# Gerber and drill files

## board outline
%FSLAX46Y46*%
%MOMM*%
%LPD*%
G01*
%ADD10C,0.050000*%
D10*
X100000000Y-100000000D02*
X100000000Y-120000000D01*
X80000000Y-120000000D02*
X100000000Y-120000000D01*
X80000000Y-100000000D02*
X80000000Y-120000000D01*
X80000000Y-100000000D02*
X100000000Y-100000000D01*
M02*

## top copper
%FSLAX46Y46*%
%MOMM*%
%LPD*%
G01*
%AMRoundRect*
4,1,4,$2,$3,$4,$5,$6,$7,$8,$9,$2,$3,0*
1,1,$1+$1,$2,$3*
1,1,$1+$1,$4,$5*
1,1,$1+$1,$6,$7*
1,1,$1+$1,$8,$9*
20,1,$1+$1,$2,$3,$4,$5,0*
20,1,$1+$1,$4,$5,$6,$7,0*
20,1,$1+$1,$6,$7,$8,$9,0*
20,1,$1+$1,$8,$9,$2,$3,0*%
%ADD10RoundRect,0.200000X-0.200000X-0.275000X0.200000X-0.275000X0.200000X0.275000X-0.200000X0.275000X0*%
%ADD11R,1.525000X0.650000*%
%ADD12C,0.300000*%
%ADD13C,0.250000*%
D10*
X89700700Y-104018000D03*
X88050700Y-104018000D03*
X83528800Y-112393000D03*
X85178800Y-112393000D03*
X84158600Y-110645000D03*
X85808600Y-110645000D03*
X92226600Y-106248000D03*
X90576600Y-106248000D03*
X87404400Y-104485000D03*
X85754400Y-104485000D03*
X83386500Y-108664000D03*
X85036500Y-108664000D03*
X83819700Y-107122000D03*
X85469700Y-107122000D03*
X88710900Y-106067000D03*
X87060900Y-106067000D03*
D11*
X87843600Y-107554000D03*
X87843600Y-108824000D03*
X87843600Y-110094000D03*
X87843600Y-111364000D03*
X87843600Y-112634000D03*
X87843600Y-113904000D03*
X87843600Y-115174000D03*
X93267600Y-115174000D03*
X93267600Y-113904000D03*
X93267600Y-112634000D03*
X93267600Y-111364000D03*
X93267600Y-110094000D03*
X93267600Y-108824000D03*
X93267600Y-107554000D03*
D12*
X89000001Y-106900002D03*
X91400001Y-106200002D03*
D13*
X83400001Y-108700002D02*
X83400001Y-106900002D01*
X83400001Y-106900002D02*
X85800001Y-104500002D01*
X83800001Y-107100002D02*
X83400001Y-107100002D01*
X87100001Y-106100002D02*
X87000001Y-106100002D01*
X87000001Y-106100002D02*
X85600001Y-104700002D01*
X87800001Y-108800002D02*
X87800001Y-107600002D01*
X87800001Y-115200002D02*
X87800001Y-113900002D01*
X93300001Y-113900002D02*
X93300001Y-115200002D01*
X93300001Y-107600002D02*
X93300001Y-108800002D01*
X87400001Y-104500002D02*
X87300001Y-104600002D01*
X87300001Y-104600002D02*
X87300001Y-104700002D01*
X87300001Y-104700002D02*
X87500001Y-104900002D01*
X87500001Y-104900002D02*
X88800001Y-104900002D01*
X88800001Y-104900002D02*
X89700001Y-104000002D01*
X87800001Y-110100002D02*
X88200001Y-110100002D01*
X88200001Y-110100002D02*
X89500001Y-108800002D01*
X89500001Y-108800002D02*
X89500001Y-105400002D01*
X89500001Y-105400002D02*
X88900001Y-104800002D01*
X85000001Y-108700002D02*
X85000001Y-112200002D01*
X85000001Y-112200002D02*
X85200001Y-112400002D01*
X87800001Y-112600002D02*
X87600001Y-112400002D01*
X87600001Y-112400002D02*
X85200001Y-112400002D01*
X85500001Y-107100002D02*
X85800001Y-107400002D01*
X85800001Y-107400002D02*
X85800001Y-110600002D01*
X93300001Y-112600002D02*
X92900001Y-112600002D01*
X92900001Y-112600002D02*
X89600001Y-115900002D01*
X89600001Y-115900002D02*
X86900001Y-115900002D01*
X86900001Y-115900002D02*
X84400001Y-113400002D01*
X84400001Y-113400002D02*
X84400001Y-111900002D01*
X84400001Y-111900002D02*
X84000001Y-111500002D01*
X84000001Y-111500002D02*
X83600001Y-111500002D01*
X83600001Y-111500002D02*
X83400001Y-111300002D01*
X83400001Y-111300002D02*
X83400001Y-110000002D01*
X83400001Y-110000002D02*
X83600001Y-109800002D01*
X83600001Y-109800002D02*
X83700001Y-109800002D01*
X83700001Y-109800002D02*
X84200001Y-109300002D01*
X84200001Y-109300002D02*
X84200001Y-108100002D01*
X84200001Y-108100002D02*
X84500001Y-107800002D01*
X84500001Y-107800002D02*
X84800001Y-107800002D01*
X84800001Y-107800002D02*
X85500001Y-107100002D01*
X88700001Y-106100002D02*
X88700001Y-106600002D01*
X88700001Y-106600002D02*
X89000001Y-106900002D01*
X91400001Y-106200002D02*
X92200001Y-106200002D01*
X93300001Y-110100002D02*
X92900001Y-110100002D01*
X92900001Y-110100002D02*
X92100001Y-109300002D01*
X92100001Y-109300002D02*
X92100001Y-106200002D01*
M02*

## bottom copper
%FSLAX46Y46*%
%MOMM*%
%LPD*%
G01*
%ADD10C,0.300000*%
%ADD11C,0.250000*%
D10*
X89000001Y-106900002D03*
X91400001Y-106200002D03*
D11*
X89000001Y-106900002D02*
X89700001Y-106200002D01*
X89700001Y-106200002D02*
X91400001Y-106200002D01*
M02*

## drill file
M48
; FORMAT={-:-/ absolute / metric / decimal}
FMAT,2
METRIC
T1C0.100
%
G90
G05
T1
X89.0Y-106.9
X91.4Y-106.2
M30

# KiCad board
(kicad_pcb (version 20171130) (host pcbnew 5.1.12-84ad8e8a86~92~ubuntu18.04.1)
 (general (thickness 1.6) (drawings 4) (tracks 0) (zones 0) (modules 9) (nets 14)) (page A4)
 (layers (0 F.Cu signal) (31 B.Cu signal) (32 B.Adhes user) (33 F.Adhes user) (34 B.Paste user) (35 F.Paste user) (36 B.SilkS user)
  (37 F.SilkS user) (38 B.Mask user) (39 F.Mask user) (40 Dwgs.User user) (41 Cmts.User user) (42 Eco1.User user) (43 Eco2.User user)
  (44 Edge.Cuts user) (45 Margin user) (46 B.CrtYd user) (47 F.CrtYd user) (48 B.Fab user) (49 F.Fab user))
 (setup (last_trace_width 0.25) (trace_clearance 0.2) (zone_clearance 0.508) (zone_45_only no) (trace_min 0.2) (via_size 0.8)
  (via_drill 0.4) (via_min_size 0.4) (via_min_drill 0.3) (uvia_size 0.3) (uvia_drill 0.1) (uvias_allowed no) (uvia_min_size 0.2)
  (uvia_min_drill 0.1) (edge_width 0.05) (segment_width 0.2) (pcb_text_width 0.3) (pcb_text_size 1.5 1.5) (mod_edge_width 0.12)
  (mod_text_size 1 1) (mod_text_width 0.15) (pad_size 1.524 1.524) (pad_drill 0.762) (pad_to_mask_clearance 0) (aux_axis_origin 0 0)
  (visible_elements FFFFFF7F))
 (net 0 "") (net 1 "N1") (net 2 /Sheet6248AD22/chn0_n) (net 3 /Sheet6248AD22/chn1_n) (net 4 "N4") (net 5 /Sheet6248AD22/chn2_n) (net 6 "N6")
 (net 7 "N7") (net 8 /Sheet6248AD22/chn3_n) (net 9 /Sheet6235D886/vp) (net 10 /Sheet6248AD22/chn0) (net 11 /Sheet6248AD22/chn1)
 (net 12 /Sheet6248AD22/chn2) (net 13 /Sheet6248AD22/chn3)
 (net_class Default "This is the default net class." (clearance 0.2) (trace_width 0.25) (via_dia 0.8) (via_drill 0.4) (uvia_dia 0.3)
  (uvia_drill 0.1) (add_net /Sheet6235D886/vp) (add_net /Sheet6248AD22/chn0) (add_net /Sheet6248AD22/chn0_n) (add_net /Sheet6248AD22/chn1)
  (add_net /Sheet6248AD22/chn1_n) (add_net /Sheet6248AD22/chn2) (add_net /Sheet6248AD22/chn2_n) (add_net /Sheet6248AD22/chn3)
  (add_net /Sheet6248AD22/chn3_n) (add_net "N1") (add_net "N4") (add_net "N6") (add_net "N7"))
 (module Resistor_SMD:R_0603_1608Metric (layer F.Cu) (at 88.875700 104.018000)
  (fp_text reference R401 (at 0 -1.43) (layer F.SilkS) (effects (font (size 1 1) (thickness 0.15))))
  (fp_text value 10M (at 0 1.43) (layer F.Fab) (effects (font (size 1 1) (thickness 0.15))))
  (pad 2 smd roundrect (at 0.825 0) (size 0.8 0.95) (layers F.Cu F.Mask F.Paste) (roundrect_rratio 0.25) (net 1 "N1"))
  (pad 1 smd roundrect (at -0.825 0) (size 0.8 0.95) (layers F.Cu F.Mask F.Paste) (roundrect_rratio 0.25) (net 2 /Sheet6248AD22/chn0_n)))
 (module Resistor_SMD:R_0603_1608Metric (layer F.Cu) (at 84.353800 112.393000)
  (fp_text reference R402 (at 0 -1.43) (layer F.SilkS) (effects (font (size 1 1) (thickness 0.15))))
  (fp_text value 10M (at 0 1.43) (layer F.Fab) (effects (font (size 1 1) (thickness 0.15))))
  (pad 1 smd roundrect (at -0.825 0) (size 0.8 0.95) (layers F.Cu F.Mask F.Paste) (roundrect_rratio 0.25) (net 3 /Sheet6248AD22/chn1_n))
  (pad 2 smd roundrect (at 0.825 0) (size 0.8 0.95) (layers F.Cu F.Mask F.Paste) (roundrect_rratio 0.25) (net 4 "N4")))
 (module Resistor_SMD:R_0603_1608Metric (layer F.Cu) (at 84.983600 110.645000)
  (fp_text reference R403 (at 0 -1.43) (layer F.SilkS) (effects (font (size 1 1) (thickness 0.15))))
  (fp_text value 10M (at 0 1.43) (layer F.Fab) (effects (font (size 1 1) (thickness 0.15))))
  (pad 1 smd roundrect (at -0.825 0) (size 0.8 0.95) (layers F.Cu F.Mask F.Paste) (roundrect_rratio 0.25) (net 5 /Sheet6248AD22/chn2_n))
  (pad 2 smd roundrect (at 0.825 0) (size 0.8 0.95) (layers F.Cu F.Mask F.Paste) (roundrect_rratio 0.25) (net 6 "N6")))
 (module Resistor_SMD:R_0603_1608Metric (layer F.Cu) (at 91.401600 106.248000)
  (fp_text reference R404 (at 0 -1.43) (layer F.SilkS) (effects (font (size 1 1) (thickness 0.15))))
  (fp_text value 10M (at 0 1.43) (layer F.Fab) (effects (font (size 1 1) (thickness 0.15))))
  (pad 2 smd roundrect (at 0.825 0) (size 0.8 0.95) (layers F.Cu F.Mask F.Paste) (roundrect_rratio 0.25) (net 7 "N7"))
  (pad 1 smd roundrect (at -0.825 0) (size 0.8 0.95) (layers F.Cu F.Mask F.Paste) (roundrect_rratio 0.25) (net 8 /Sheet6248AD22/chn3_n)))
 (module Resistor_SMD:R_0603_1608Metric (layer F.Cu) (at 86.579400 104.485000)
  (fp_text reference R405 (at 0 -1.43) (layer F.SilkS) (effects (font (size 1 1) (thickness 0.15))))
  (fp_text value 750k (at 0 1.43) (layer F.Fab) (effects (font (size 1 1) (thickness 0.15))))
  (pad 2 smd roundrect (at 0.825 0) (size 0.8 0.95) (layers F.Cu F.Mask F.Paste) (roundrect_rratio 0.25) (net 1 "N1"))
  (pad 1 smd roundrect (at -0.825 0) (size 0.8 0.95) (layers F.Cu F.Mask F.Paste) (roundrect_rratio 0.25) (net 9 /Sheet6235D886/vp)))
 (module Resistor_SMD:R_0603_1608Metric (layer F.Cu) (at 84.211500 108.664000)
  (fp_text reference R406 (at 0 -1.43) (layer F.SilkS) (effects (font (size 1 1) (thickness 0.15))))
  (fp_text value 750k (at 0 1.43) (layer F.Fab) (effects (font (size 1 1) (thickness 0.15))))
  (pad 1 smd roundrect (at -0.825 0) (size 0.8 0.95) (layers F.Cu F.Mask F.Paste) (roundrect_rratio 0.25) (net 9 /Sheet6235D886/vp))
  (pad 2 smd roundrect (at 0.825 0) (size 0.8 0.95) (layers F.Cu F.Mask F.Paste) (roundrect_rratio 0.25) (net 4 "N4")))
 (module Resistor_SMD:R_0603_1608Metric (layer F.Cu) (at 84.644700 107.122000)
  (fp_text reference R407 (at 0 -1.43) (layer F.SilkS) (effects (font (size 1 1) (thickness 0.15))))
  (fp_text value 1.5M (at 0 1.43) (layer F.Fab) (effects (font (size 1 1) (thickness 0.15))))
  (pad 1 smd roundrect (at -0.825 0) (size 0.8 0.95) (layers F.Cu F.Mask F.Paste) (roundrect_rratio 0.25) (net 9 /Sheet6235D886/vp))
  (pad 2 smd roundrect (at 0.825 0) (size 0.8 0.95) (layers F.Cu F.Mask F.Paste) (roundrect_rratio 0.25) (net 6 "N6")))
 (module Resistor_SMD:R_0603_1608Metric (layer F.Cu) (at 87.885900 106.067000)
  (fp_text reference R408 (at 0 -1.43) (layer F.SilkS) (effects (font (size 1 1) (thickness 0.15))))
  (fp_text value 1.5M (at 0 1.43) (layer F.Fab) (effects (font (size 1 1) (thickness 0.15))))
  (pad 2 smd roundrect (at 0.825 0) (size 0.8 0.95) (layers F.Cu F.Mask F.Paste) (roundrect_rratio 0.25) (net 7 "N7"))
  (pad 1 smd roundrect (at -0.825 0) (size 0.8 0.95) (layers F.Cu F.Mask F.Paste) (roundrect_rratio 0.25) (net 9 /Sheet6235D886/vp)))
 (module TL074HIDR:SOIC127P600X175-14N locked (layer F.Cu) (at 90.555600 111.364000)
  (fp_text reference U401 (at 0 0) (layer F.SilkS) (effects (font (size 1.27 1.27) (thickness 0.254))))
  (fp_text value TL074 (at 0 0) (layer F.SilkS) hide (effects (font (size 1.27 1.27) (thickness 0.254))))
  (pad 1 smd rect (at -2.712 -3.81 90.000000) (size 0.65 1.525) (layers F.Cu F.Mask F.Paste) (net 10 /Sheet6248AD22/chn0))
  (pad 2 smd rect (at -2.712 -2.54 90.000000) (size 0.65 1.525) (layers F.Cu F.Mask F.Paste) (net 10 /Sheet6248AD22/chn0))
  (pad 3 smd rect (at -2.712 -1.27 90.000000) (size 0.65 1.525) (layers F.Cu F.Mask F.Paste) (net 1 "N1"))
  (pad 4 smd rect (at -2.712 0 90.000000) (size 0.65 1.525) (layers F.Cu F.Mask F.Paste))
  (pad 5 smd rect (at -2.712 1.27 90.000000) (size 0.65 1.525) (layers F.Cu F.Mask F.Paste) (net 4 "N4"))
  (pad 6 smd rect (at -2.712 2.54 90.000000) (size 0.65 1.525) (layers F.Cu F.Mask F.Paste) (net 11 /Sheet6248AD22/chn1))
  (pad 7 smd rect (at -2.712 3.81 90.000000) (size 0.65 1.525) (layers F.Cu F.Mask F.Paste) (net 11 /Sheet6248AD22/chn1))
  (pad 8 smd rect (at 2.712 3.81 90.000000) (size 0.65 1.525) (layers F.Cu F.Mask F.Paste) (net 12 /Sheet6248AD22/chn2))
  (pad 9 smd rect (at 2.712 2.54 90.000000) (size 0.65 1.525) (layers F.Cu F.Mask F.Paste) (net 12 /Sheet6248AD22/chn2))
  (pad 10 smd rect (at 2.712 1.27 90.000000) (size 0.65 1.525) (layers F.Cu F.Mask F.Paste) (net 6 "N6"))
  (pad 11 smd rect (at 2.712 0 90.000000) (size 0.65 1.525) (layers F.Cu F.Mask F.Paste))
  (pad 12 smd rect (at 2.712 -1.27 90.000000) (size 0.65 1.525) (layers F.Cu F.Mask F.Paste) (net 7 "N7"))
  (pad 13 smd rect (at 2.712 -2.54 90.000000) (size 0.65 1.525) (layers F.Cu F.Mask F.Paste) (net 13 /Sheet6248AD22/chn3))
  (pad 14 smd rect (at 2.712 -3.81 90.000000) (size 0.65 1.525) (layers F.Cu F.Mask F.Paste) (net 13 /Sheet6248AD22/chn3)))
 (gr_line (start 100 100) (end 100 120) (layer Edge.Cuts) (width 0.05))
 (gr_line (start 80 120) (end 100 120) (layer Edge.Cuts) (width 0.05))
 (gr_line (start 80 100) (end 80 120) (layer Edge.Cuts) (width 0.05))
 (gr_line (start 80 100) (end 100 100) (layer Edge.Cuts) (width 0.05))
 (segment (start 83.400001 108.700002) (end 83.400001 106.900002) (width 0.250000) (layer F.Cu) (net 9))
 (segment (start 83.400001 106.900002) (end 85.800001 104.500002) (width 0.250000) (layer F.Cu) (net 9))
 (segment (start 83.800001 107.100002) (end 83.400001 107.100002) (width 0.250000) (layer F.Cu) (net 9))
 (segment (start 87.100001 106.100002) (end 87.000001 106.100002) (width 0.250000) (layer F.Cu) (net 9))
 (segment (start 87.000001 106.100002) (end 85.600001 104.700002) (width 0.250000) (layer F.Cu) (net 9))
 (segment (start 87.800001 108.800002) (end 87.800001 107.600002) (width 0.250000) (layer F.Cu) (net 10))
 (segment (start 87.800001 115.200002) (end 87.800001 113.900002) (width 0.250000) (layer F.Cu) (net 11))
 (segment (start 93.300001 113.900002) (end 93.300001 115.200002) (width 0.250000) (layer F.Cu) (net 12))
 (segment (start 93.300001 107.600002) (end 93.300001 108.800002) (width 0.250000) (layer F.Cu) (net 13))
 (segment (start 87.400001 104.500002) (end 87.300001 104.600002) (width 0.250000) (layer F.Cu) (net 1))
 (segment (start 87.300001 104.600002) (end 87.300001 104.700002) (width 0.250000) (layer F.Cu) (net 1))
 (segment (start 87.300001 104.700002) (end 87.500001 104.900002) (width 0.250000) (layer F.Cu) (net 1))
 (segment (start 87.500001 104.900002) (end 88.800001 104.900002) (width 0.250000) (layer F.Cu) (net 1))
 (segment (start 88.800001 104.900002) (end 89.700001 104.000002) (width 0.250000) (layer F.Cu) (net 1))
 (segment (start 87.800001 110.100002) (end 88.200001 110.100002) (width 0.250000) (layer F.Cu) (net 1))
 (segment (start 88.200001 110.100002) (end 89.500001 108.800002) (width 0.250000) (layer F.Cu) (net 1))
 (segment (start 89.500001 108.800002) (end 89.500001 105.400002) (width 0.250000) (layer F.Cu) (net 1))
 (segment (start 89.500001 105.400002) (end 88.900001 104.800002) (width 0.250000) (layer F.Cu) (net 1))
 (segment (start 85.000001 108.700002) (end 85.000001 112.200002) (width 0.250000) (layer F.Cu) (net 4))
 (segment (start 85.000001 112.200002) (end 85.200001 112.400002) (width 0.250000) (layer F.Cu) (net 4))
 (segment (start 87.800001 112.600002) (end 87.600001 112.400002) (width 0.250000) (layer F.Cu) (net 4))
 (segment (start 87.600001 112.400002) (end 85.200001 112.400002) (width 0.250000) (layer F.Cu) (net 4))
 (segment (start 85.500001 107.100002) (end 85.800001 107.400002) (width 0.250000) (layer F.Cu) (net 6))
 (segment (start 85.800001 107.400002) (end 85.800001 110.600002) (width 0.250000) (layer F.Cu) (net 6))
 (segment (start 93.300001 112.600002) (end 92.900001 112.600002) (width 0.250000) (layer F.Cu) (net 6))
 (segment (start 92.900001 112.600002) (end 89.600001 115.900002) (width 0.250000) (layer F.Cu) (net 6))
 (segment (start 89.600001 115.900002) (end 86.900001 115.900002) (width 0.250000) (layer F.Cu) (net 6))
 (segment (start 86.900001 115.900002) (end 84.400001 113.400002) (width 0.250000) (layer F.Cu) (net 6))
 (segment (start 84.400001 113.400002) (end 84.400001 111.900002) (width 0.250000) (layer F.Cu) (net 6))
 (segment (start 84.400001 111.900002) (end 84.000001 111.500002) (width 0.250000) (layer F.Cu) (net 6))
 (segment (start 84.000001 111.500002) (end 83.600001 111.500002) (width 0.250000) (layer F.Cu) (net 6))
 (segment (start 83.600001 111.500002) (end 83.400001 111.300002) (width 0.250000) (layer F.Cu) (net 6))
 (segment (start 83.400001 111.300002) (end 83.400001 110.000002) (width 0.250000) (layer F.Cu) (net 6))
 (segment (start 83.400001 110.000002) (end 83.600001 109.800002) (width 0.250000) (layer F.Cu) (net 6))
 (segment (start 83.600001 109.800002) (end 83.700001 109.800002) (width 0.250000) (layer F.Cu) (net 6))
 (segment (start 83.700001 109.800002) (end 84.200001 109.300002) (width 0.250000) (layer F.Cu) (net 6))
 (segment (start 84.200001 109.300002) (end 84.200001 108.100002) (width 0.250000) (layer F.Cu) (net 6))
 (segment (start 84.200001 108.100002) (end 84.500001 107.800002) (width 0.250000) (layer F.Cu) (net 6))
 (segment (start 84.500001 107.800002) (end 84.800001 107.800002) (width 0.250000) (layer F.Cu) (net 6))
 (segment (start 84.800001 107.800002) (end 85.500001 107.100002) (width 0.250000) (layer F.Cu) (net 6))
 (segment (start 88.700001 106.100002) (end 88.700001 106.600002) (width 0.250000) (layer F.Cu) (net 7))
 (segment (start 88.700001 106.600002) (end 89.000001 106.900002) (width 0.250000) (layer F.Cu) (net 7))
 (segment (start 89.000001 106.900002) (end 89.700001 106.200002) (width 0.250000) (layer B.Cu) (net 7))
 (segment (start 89.700001 106.200002) (end 91.400001 106.200002) (width 0.250000) (layer B.Cu) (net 7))
 (segment (start 91.400001 106.200002) (end 92.200001 106.200002) (width 0.250000) (layer F.Cu) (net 7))
 (segment (start 93.300001 110.100002) (end 92.900001 110.100002) (width 0.250000) (layer F.Cu) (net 7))
 (segment (start 92.900001 110.100002) (end 92.100001 109.300002) (width 0.250000) (layer F.Cu) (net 7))
 (segment (start 92.100001 109.300002) (end 92.100001 106.200002) (width 0.250000) (layer F.Cu) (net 7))
 (via micro (at 89.000001 106.900002) (size 0.300000) (drill 0.100000) (layers F.Cu B.Cu) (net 7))
 (via micro (at 91.400001 106.200002) (size 0.300000) (drill 0.100000) (layers F.Cu B.Cu) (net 7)))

